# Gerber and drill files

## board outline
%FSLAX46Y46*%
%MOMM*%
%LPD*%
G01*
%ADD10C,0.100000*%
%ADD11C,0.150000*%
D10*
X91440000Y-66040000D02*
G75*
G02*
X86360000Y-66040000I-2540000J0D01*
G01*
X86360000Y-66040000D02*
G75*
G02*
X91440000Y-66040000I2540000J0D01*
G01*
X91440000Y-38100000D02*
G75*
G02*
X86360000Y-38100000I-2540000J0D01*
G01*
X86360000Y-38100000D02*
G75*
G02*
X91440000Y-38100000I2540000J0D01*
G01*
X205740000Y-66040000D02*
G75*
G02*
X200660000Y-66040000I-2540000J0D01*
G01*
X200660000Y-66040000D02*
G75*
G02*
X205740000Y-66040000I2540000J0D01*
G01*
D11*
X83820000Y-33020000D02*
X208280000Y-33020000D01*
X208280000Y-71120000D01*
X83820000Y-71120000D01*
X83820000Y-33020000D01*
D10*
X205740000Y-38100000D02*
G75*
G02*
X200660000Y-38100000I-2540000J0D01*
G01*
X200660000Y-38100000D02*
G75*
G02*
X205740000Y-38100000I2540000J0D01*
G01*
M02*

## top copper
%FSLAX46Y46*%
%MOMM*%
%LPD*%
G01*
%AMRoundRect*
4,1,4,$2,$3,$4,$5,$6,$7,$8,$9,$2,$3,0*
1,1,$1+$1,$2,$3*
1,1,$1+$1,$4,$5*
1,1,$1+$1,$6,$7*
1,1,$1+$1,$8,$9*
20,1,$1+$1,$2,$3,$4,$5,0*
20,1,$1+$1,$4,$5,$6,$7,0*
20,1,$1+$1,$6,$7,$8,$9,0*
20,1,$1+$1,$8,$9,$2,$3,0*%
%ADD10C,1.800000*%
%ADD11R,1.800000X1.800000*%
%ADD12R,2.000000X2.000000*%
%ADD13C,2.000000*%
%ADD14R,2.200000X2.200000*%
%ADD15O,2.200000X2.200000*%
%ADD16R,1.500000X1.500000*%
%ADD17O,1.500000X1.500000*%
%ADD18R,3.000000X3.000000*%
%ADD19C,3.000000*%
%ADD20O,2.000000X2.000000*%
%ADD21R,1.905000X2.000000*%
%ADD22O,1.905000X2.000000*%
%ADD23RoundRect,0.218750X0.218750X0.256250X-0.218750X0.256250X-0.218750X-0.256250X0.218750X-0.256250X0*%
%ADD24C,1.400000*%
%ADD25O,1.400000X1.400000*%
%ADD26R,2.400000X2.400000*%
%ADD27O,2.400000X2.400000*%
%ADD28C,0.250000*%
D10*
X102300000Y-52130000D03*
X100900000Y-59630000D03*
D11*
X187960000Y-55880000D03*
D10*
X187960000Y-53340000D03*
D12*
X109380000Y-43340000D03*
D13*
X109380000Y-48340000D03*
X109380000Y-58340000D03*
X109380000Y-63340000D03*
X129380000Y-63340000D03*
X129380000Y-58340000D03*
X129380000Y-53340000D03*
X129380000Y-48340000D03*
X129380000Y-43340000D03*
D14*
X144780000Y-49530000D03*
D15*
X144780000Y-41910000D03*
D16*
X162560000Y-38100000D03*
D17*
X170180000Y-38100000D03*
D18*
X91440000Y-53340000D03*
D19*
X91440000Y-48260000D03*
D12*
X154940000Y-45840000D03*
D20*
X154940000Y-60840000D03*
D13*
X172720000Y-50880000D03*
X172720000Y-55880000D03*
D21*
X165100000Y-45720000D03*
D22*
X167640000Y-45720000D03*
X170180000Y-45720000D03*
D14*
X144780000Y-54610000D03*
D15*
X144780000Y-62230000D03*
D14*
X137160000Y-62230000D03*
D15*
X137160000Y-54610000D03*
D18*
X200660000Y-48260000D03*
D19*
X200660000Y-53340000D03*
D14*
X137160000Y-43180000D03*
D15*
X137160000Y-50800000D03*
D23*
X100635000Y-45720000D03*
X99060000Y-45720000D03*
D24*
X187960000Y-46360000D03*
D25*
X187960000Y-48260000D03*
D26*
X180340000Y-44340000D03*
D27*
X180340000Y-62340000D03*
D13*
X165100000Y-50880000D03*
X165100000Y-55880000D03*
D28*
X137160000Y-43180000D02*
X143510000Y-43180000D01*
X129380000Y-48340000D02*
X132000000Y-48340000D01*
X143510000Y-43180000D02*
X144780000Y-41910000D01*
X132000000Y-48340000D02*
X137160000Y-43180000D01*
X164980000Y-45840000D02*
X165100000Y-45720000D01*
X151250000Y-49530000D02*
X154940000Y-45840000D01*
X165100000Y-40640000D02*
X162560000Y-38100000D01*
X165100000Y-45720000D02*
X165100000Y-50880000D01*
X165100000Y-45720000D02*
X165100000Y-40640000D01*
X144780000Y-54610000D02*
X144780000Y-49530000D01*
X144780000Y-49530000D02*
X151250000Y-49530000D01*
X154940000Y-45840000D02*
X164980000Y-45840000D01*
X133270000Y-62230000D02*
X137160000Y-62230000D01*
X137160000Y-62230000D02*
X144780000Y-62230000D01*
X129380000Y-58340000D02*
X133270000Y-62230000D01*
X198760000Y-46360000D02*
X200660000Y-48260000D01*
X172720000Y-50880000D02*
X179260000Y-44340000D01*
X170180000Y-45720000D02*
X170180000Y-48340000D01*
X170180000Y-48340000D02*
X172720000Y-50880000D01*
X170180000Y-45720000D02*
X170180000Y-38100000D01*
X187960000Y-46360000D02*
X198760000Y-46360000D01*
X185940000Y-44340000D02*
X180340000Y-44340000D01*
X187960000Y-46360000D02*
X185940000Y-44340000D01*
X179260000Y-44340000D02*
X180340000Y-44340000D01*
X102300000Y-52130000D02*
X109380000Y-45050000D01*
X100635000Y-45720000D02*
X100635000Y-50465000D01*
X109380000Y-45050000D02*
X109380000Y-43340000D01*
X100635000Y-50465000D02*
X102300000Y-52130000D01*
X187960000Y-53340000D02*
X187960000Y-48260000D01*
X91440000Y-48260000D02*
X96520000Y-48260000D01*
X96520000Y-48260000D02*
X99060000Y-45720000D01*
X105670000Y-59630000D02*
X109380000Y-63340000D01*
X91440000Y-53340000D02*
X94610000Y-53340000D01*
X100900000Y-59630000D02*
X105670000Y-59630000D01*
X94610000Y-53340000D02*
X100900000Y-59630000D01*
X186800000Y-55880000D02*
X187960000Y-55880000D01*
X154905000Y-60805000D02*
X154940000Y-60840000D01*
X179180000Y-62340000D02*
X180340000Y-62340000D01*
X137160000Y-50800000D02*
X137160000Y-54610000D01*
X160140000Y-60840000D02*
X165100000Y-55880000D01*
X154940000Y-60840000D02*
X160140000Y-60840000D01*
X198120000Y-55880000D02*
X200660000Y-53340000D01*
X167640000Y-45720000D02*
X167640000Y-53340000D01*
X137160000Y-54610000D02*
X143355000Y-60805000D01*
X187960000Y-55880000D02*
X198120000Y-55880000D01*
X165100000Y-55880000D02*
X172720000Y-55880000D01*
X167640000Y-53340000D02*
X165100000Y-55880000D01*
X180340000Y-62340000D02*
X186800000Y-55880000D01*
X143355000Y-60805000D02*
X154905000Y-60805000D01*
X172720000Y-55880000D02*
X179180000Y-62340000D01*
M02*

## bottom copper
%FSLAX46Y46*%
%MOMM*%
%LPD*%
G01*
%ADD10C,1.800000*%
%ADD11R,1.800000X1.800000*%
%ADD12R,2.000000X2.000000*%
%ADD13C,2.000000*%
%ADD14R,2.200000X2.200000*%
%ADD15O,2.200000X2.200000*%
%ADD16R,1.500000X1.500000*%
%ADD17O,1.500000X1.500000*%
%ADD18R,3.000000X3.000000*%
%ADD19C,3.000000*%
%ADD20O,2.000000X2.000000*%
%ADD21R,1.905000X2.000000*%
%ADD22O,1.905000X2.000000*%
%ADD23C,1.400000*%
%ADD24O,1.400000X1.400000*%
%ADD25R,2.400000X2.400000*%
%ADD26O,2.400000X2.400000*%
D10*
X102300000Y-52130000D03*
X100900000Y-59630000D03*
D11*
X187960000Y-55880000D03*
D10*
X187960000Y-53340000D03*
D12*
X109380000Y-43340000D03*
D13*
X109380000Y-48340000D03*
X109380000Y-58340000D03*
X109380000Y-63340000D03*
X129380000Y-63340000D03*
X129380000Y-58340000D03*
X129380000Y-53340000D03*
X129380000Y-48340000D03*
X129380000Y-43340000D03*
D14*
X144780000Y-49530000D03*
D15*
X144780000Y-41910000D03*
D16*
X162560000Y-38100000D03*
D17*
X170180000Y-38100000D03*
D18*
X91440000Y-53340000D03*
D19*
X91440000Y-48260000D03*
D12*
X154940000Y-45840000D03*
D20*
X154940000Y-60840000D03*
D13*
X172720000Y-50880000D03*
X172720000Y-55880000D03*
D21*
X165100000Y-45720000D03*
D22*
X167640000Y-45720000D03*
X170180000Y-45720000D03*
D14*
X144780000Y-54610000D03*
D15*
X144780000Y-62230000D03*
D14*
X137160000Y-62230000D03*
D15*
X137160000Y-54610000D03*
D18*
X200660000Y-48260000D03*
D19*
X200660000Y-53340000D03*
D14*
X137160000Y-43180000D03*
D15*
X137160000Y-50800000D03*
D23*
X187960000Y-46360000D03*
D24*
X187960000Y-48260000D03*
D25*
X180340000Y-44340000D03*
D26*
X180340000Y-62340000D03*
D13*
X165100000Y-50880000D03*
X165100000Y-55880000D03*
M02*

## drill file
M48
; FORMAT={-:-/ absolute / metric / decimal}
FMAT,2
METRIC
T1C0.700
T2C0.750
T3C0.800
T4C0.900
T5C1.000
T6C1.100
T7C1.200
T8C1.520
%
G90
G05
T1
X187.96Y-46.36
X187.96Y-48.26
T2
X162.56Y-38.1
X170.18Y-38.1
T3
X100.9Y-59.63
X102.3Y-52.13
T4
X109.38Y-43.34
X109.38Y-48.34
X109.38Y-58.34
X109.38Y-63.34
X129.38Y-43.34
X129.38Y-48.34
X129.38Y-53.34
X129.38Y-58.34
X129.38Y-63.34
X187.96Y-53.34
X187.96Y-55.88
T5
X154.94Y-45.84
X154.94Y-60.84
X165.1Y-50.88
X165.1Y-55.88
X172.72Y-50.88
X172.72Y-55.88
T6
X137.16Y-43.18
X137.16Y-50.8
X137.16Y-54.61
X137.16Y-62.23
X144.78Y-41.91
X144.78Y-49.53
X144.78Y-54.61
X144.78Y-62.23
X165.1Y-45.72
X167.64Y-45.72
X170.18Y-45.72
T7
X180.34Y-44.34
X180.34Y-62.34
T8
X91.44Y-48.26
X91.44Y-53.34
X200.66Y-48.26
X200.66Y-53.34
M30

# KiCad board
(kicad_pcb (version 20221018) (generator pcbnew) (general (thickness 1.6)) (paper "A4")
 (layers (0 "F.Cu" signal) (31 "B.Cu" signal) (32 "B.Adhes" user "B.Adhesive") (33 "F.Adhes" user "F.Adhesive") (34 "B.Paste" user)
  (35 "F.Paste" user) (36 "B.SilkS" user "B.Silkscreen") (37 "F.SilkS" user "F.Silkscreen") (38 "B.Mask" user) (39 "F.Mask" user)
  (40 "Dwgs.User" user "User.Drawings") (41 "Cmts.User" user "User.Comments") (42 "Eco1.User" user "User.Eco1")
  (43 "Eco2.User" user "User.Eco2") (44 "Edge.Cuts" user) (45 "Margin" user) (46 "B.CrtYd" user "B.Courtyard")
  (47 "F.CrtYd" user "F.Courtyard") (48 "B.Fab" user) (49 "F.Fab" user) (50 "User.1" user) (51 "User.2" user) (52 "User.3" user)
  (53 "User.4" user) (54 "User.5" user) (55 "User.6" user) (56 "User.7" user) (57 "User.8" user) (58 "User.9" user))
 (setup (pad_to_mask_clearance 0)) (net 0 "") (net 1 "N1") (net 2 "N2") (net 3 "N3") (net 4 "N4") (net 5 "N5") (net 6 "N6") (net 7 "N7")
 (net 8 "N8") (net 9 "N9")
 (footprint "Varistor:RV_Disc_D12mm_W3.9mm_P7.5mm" (layer "F.Cu") (at 102.3 52.13 -90)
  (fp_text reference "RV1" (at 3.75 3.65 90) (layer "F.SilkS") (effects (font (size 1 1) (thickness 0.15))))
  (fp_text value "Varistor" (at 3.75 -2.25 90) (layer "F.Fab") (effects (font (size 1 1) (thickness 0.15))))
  (pad "1" thru_hole circle (at 0 0 270) (size 1.8 1.8) (drill 0.8) (layers "*.Cu" "*.Mask") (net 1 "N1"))
  (pad "2" thru_hole circle (at 7.5 1.4 270) (size 1.8 1.8) (drill 0.8) (layers "*.Cu" "*.Mask") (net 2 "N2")))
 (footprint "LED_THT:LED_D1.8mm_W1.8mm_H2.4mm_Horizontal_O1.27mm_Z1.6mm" (layer "F.Cu") (at 187.96 55.88 90)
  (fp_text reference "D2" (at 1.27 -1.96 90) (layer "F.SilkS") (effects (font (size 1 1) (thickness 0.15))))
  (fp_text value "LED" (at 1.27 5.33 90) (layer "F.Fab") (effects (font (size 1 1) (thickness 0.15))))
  (pad "1" thru_hole rect (at 0 0 90) (size 1.8 1.8) (drill 0.9) (layers "*.Cu" "*.Mask") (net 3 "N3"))
  (pad "2" thru_hole circle (at 2.54 0 90) (size 1.8 1.8) (drill 0.9) (layers "*.Cu" "*.Mask") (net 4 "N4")))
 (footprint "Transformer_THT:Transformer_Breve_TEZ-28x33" (layer "F.Cu") (at 109.38 43.34 -90)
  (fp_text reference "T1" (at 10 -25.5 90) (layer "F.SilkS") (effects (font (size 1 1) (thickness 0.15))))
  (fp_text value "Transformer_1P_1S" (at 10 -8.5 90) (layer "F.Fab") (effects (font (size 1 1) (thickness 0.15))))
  (pad "1" thru_hole rect (at 0 0 270) (size 2 2) (drill 0.9) (layers "*.Cu" "*.Mask") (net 1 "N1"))
  (pad "2" thru_hole circle (at 5 0 270) (size 2 2) (drill 0.9) (layers "*.Cu" "*.Mask"))
  (pad "4" thru_hole circle (at 15 0 270) (size 2 2) (drill 0.9) (layers "*.Cu" "*.Mask"))
  (pad "5" thru_hole circle (at 20 0 270) (size 2 2) (drill 0.9) (layers "*.Cu" "*.Mask") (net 2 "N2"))
  (pad "6" thru_hole circle (at 20 -20 270) (size 2 2) (drill 0.9) (layers "*.Cu" "*.Mask"))
  (pad "7" thru_hole circle (at 15 -20 270) (size 2 2) (drill 0.9) (layers "*.Cu" "*.Mask") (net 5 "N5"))
  (pad "8" thru_hole circle (at 10 -20 270) (size 2 2) (drill 0.9) (layers "*.Cu" "*.Mask"))
  (pad "9" thru_hole circle (at 5 -20 270) (size 2 2) (drill 0.9) (layers "*.Cu" "*.Mask") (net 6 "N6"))
  (pad "10" thru_hole circle (at 0 -20 270) (size 2 2) (drill 0.9) (layers "*.Cu" "*.Mask")))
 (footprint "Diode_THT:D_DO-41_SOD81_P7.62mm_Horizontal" (layer "F.Cu") (at 144.78 49.53 90)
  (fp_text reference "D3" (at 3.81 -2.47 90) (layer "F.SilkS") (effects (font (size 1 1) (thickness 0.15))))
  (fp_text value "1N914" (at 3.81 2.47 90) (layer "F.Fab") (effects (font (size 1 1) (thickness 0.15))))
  (pad "1" thru_hole rect (at 0 0 90) (size 2.2 2.2) (drill 1.1) (layers "*.Cu" "*.Mask") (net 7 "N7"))
  (pad "2" thru_hole oval (at 7.62 0 90) (size 2.2 2.2) (drill 1.1) (layers "*.Cu" "*.Mask") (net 6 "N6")))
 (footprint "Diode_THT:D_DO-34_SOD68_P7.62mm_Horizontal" (layer "F.Cu") (at 162.56 38.1)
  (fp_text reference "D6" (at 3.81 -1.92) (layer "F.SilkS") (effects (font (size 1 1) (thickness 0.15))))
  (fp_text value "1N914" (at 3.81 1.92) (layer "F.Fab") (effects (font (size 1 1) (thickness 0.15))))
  (pad "1" thru_hole rect (at 0 0) (size 1.5 1.5) (drill 0.75) (layers "*.Cu" "*.Mask") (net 7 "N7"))
  (pad "2" thru_hole oval (at 7.62 0) (size 1.5 1.5) (drill 0.75) (layers "*.Cu" "*.Mask") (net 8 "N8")))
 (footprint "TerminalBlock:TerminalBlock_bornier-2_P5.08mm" (layer "F.Cu") (at 91.44 53.34 90)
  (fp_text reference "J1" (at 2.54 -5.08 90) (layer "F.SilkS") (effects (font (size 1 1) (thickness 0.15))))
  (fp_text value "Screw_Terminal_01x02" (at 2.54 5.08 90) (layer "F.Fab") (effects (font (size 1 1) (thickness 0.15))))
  (pad "1" thru_hole rect (at 0 0 90) (size 3 3) (drill 1.52) (layers "*.Cu" "*.Mask") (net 2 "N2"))
  (pad "2" thru_hole circle (at 5.08 0 90) (size 3 3) (drill 1.52) (layers "*.Cu" "*.Mask") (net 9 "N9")))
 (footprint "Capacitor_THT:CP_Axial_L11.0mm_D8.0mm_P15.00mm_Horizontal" (layer "F.Cu") (at 154.94 45.84 -90)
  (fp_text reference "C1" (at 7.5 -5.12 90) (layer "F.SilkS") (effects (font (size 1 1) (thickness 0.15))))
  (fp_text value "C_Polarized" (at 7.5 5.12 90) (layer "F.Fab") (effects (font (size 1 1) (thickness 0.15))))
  (pad "1" thru_hole rect (at 0 0 270) (size 2 2) (drill 1) (layers "*.Cu" "*.Mask") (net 7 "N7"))
  (pad "2" thru_hole oval (at 15 0 270) (size 2 2) (drill 1) (layers "*.Cu" "*.Mask") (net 3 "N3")))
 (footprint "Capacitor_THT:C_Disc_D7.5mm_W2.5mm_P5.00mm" (layer "F.Cu") (at 172.72 50.88 -90)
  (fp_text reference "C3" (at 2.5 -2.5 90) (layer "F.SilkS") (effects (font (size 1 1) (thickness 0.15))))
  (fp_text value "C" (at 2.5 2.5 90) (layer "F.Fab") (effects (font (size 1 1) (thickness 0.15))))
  (pad "1" thru_hole circle (at 0 0 270) (size 2 2) (drill 1) (layers "*.Cu" "*.Mask") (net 8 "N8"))
  (pad "2" thru_hole circle (at 5 0 270) (size 2 2) (drill 1) (layers "*.Cu" "*.Mask") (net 3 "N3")))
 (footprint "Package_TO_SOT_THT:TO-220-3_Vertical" (layer "F.Cu") (at 165.1 45.72)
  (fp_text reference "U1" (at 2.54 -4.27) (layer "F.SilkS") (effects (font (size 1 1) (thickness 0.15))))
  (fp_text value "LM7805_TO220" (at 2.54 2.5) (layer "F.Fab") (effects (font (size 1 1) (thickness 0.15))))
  (pad "1" thru_hole rect (at 0 0) (size 1.905 2) (drill 1.1) (layers "*.Cu" "*.Mask") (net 7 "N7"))
  (pad "2" thru_hole oval (at 2.54 0) (size 1.905 2) (drill 1.1) (layers "*.Cu" "*.Mask") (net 3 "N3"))
  (pad "3" thru_hole oval (at 5.08 0) (size 1.905 2) (drill 1.1) (layers "*.Cu" "*.Mask") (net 8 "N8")))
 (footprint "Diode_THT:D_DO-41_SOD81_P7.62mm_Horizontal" (layer "F.Cu") (at 144.78 54.61 -90)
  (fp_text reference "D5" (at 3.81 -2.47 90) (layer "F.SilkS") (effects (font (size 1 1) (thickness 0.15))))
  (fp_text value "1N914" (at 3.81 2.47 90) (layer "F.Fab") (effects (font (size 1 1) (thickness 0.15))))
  (pad "1" thru_hole rect (at 0 0 270) (size 2.2 2.2) (drill 1.1) (layers "*.Cu" "*.Mask") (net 7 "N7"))
  (pad "2" thru_hole oval (at 7.62 0 270) (size 2.2 2.2) (drill 1.1) (layers "*.Cu" "*.Mask") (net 5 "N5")))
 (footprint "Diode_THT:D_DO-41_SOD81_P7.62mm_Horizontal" (layer "F.Cu") (at 137.16 62.23 90)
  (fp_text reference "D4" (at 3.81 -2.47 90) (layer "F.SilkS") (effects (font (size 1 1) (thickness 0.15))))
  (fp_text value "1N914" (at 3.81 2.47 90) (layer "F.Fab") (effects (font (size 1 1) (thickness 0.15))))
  (pad "1" thru_hole rect (at 0 0 90) (size 2.2 2.2) (drill 1.1) (layers "*.Cu" "*.Mask") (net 5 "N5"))
  (pad "2" thru_hole oval (at 7.62 0 90) (size 2.2 2.2) (drill 1.1) (layers "*.Cu" "*.Mask") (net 3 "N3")))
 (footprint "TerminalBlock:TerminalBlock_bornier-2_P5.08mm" (layer "F.Cu") (at 200.66 48.26 -90)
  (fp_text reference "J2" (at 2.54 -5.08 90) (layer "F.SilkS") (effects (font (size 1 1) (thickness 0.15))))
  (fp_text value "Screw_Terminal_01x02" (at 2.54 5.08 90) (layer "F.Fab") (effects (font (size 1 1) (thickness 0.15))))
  (pad "1" thru_hole rect (at 0 0 270) (size 3 3) (drill 1.52) (layers "*.Cu" "*.Mask") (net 8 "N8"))
  (pad "2" thru_hole circle (at 5.08 0 270) (size 3 3) (drill 1.52) (layers "*.Cu" "*.Mask") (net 3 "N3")))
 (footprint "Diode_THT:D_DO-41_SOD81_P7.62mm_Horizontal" (layer "F.Cu") (at 137.16 43.18 -90)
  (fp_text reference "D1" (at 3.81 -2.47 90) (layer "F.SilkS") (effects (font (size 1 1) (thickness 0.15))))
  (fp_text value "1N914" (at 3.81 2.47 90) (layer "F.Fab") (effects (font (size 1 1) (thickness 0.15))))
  (pad "1" thru_hole rect (at 0 0 270) (size 2.2 2.2) (drill 1.1) (layers "*.Cu" "*.Mask") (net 6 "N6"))
  (pad "2" thru_hole oval (at 7.62 0 270) (size 2.2 2.2) (drill 1.1) (layers "*.Cu" "*.Mask") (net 3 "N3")))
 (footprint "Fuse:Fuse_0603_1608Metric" (layer "F.Cu") (at 99.8475 45.72 180)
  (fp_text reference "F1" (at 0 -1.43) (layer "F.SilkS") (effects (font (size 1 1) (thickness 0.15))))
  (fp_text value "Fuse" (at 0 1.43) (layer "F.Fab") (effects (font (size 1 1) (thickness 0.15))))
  (pad "1" smd roundrect (at -0.7875 0 180) (size 0.875 0.95) (layers "F.Cu" "F.Paste" "F.Mask") (roundrect_rratio 0.25) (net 1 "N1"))
  (pad "2" smd roundrect (at 0.7875 0 180) (size 0.875 0.95) (layers "F.Cu" "F.Paste" "F.Mask") (roundrect_rratio 0.25) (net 9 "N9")))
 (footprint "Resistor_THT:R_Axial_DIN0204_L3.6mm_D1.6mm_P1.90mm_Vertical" (layer "F.Cu") (at 187.96 46.36 -90)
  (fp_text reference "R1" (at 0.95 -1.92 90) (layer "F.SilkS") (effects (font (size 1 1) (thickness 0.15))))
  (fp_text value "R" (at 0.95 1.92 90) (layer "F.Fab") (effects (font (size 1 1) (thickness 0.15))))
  (pad "1" thru_hole circle (at 0 0 270) (size 1.4 1.4) (drill 0.7) (layers "*.Cu" "*.Mask") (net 8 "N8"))
  (pad "2" thru_hole oval (at 1.9 0 270) (size 1.4 1.4) (drill 0.7) (layers "*.Cu" "*.Mask") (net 4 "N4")))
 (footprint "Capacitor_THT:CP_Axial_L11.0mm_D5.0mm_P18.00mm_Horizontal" (layer "F.Cu") (at 180.34 44.34 -90)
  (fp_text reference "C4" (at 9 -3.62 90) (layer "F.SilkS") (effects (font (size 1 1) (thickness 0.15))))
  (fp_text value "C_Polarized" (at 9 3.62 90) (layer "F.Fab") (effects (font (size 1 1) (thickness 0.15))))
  (pad "1" thru_hole rect (at 0 0 270) (size 2.4 2.4) (drill 1.2) (layers "*.Cu" "*.Mask") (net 8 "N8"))
  (pad "2" thru_hole oval (at 18 0 270) (size 2.4 2.4) (drill 1.2) (layers "*.Cu" "*.Mask") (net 3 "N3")))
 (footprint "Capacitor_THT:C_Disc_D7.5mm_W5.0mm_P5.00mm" (layer "F.Cu") (at 165.1 50.88 -90)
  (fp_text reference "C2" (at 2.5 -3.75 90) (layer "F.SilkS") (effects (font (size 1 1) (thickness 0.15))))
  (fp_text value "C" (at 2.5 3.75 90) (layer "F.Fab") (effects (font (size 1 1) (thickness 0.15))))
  (pad "1" thru_hole circle (at 0 0 270) (size 2 2) (drill 1) (layers "*.Cu" "*.Mask") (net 7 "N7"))
  (pad "2" thru_hole circle (at 5 0 270) (size 2 2) (drill 1) (layers "*.Cu" "*.Mask") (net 3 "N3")))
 (gr_circle (center 88.9 66.04) (end 86.36 66.04) (stroke (width 0.1) (type default)) (fill none) (layer "Edge.Cuts"))
 (gr_circle (center 88.9 38.1) (end 91.44 38.1) (stroke (width 0.1) (type default)) (fill none) (layer "Edge.Cuts"))
 (gr_circle (center 203.2 66.04) (end 200.66 66.04) (stroke (width 0.1) (type default)) (fill none) (layer "Edge.Cuts"))
 (gr_rect (start 83.82 33.02) (end 208.28 71.12) (stroke (width 0.15) (type default)) (fill none) (layer "Edge.Cuts"))
 (gr_circle (center 203.2 38.1) (end 205.74 38.1) (stroke (width 0.1) (type default)) (fill none) (layer "Edge.Cuts"))
 (segment (start 137.16 43.18) (end 143.51 43.18) (width 0.25) (layer "F.Cu") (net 6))
 (segment (start 129.38 48.34) (end 132 48.34) (width 0.25) (layer "F.Cu") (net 6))
 (segment (start 143.51 43.18) (end 144.78 41.91) (width 0.25) (layer "F.Cu") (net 6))
 (segment (start 132 48.34) (end 137.16 43.18) (width 0.25) (layer "F.Cu") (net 6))
 (segment (start 164.98 45.84) (end 165.1 45.72) (width 0.25) (layer "F.Cu") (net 7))
 (segment (start 151.25 49.53) (end 154.94 45.84) (width 0.25) (layer "F.Cu") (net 7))
 (segment (start 165.1 40.64) (end 162.56 38.1) (width 0.25) (layer "F.Cu") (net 7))
 (segment (start 165.1 45.72) (end 165.1 50.88) (width 0.25) (layer "F.Cu") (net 7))
 (segment (start 165.1 45.72) (end 165.1 40.64) (width 0.25) (layer "F.Cu") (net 7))
 (segment (start 144.78 54.61) (end 144.78 49.53) (width 0.25) (layer "F.Cu") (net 7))
 (segment (start 144.78 49.53) (end 151.25 49.53) (width 0.25) (layer "F.Cu") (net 7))
 (segment (start 154.94 45.84) (end 164.98 45.84) (width 0.25) (layer "F.Cu") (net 7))
 (segment (start 133.27 62.23) (end 137.16 62.23) (width 0.25) (layer "F.Cu") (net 5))
 (segment (start 137.16 62.23) (end 144.78 62.23) (width 0.25) (layer "F.Cu") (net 5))
 (segment (start 129.38 58.34) (end 133.27 62.23) (width 0.25) (layer "F.Cu") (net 5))
 (segment (start 198.76 46.36) (end 200.66 48.26) (width 0.25) (layer "F.Cu") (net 8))
 (segment (start 172.72 50.88) (end 179.26 44.34) (width 0.25) (layer "F.Cu") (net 8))
 (segment (start 170.18 45.72) (end 170.18 48.34) (width 0.25) (layer "F.Cu") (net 8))
 (segment (start 170.18 48.34) (end 172.72 50.88) (width 0.25) (layer "F.Cu") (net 8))
 (segment (start 170.18 45.72) (end 170.18 38.1) (width 0.25) (layer "F.Cu") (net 8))
 (segment (start 187.96 46.36) (end 198.76 46.36) (width 0.25) (layer "F.Cu") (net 8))
 (segment (start 185.94 44.34) (end 180.34 44.34) (width 0.25) (layer "F.Cu") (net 8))
 (segment (start 187.96 46.36) (end 185.94 44.34) (width 0.25) (layer "F.Cu") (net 8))
 (segment (start 179.26 44.34) (end 180.34 44.34) (width 0.25) (layer "F.Cu") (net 8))
 (segment (start 102.3 52.13) (end 109.38 45.05) (width 0.25) (layer "F.Cu") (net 1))
 (segment (start 100.635 45.72) (end 100.635 50.465) (width 0.25) (layer "F.Cu") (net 1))
 (segment (start 109.38 45.05) (end 109.38 43.34) (width 0.25) (layer "F.Cu") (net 1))
 (segment (start 100.635 50.465) (end 102.3 52.13) (width 0.25) (layer "F.Cu") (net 1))
 (segment (start 187.96 53.34) (end 187.96 48.26) (width 0.25) (layer "F.Cu") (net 4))
 (segment (start 91.44 48.26) (end 96.52 48.26) (width 0.25) (layer "F.Cu") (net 9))
 (segment (start 96.52 48.26) (end 99.06 45.72) (width 0.25) (layer "F.Cu") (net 9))
 (segment (start 105.67 59.63) (end 109.38 63.34) (width 0.25) (layer "F.Cu") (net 2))
 (segment (start 91.44 53.34) (end 94.61 53.34) (width 0.25) (layer "F.Cu") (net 2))
 (segment (start 100.9 59.63) (end 105.67 59.63) (width 0.25) (layer "F.Cu") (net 2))
 (segment (start 94.61 53.34) (end 100.9 59.63) (width 0.25) (layer "F.Cu") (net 2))
 (segment (start 186.8 55.88) (end 187.96 55.88) (width 0.25) (layer "F.Cu") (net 3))
 (segment (start 154.905 60.805) (end 154.94 60.84) (width 0.25) (layer "F.Cu") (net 3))
 (segment (start 179.18 62.34) (end 180.34 62.34) (width 0.25) (layer "F.Cu") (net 3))
 (segment (start 137.16 50.8) (end 137.16 54.61) (width 0.25) (layer "F.Cu") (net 3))
 (segment (start 160.14 60.84) (end 165.1 55.88) (width 0.25) (layer "F.Cu") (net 3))
 (segment (start 154.94 60.84) (end 160.14 60.84) (width 0.25) (layer "F.Cu") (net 3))
 (segment (start 198.12 55.88) (end 200.66 53.34) (width 0.25) (layer "F.Cu") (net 3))
 (segment (start 167.64 45.72) (end 167.64 53.34) (width 0.25) (layer "F.Cu") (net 3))
 (segment (start 137.16 54.61) (end 143.355 60.805) (width 0.25) (layer "F.Cu") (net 3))
 (segment (start 187.96 55.88) (end 198.12 55.88) (width 0.25) (layer "F.Cu") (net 3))
 (segment (start 165.1 55.88) (end 172.72 55.88) (width 0.25) (layer "F.Cu") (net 3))
 (segment (start 167.64 53.34) (end 165.1 55.88) (width 0.25) (layer "F.Cu") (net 3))
 (segment (start 180.34 62.34) (end 186.8 55.88) (width 0.25) (layer "F.Cu") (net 3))
 (segment (start 143.355 60.805) (end 154.905 60.805) (width 0.25) (layer "F.Cu") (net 3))
 (segment (start 172.72 55.88) (end 179.18 62.34) (width 0.25) (layer "F.Cu") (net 3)))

